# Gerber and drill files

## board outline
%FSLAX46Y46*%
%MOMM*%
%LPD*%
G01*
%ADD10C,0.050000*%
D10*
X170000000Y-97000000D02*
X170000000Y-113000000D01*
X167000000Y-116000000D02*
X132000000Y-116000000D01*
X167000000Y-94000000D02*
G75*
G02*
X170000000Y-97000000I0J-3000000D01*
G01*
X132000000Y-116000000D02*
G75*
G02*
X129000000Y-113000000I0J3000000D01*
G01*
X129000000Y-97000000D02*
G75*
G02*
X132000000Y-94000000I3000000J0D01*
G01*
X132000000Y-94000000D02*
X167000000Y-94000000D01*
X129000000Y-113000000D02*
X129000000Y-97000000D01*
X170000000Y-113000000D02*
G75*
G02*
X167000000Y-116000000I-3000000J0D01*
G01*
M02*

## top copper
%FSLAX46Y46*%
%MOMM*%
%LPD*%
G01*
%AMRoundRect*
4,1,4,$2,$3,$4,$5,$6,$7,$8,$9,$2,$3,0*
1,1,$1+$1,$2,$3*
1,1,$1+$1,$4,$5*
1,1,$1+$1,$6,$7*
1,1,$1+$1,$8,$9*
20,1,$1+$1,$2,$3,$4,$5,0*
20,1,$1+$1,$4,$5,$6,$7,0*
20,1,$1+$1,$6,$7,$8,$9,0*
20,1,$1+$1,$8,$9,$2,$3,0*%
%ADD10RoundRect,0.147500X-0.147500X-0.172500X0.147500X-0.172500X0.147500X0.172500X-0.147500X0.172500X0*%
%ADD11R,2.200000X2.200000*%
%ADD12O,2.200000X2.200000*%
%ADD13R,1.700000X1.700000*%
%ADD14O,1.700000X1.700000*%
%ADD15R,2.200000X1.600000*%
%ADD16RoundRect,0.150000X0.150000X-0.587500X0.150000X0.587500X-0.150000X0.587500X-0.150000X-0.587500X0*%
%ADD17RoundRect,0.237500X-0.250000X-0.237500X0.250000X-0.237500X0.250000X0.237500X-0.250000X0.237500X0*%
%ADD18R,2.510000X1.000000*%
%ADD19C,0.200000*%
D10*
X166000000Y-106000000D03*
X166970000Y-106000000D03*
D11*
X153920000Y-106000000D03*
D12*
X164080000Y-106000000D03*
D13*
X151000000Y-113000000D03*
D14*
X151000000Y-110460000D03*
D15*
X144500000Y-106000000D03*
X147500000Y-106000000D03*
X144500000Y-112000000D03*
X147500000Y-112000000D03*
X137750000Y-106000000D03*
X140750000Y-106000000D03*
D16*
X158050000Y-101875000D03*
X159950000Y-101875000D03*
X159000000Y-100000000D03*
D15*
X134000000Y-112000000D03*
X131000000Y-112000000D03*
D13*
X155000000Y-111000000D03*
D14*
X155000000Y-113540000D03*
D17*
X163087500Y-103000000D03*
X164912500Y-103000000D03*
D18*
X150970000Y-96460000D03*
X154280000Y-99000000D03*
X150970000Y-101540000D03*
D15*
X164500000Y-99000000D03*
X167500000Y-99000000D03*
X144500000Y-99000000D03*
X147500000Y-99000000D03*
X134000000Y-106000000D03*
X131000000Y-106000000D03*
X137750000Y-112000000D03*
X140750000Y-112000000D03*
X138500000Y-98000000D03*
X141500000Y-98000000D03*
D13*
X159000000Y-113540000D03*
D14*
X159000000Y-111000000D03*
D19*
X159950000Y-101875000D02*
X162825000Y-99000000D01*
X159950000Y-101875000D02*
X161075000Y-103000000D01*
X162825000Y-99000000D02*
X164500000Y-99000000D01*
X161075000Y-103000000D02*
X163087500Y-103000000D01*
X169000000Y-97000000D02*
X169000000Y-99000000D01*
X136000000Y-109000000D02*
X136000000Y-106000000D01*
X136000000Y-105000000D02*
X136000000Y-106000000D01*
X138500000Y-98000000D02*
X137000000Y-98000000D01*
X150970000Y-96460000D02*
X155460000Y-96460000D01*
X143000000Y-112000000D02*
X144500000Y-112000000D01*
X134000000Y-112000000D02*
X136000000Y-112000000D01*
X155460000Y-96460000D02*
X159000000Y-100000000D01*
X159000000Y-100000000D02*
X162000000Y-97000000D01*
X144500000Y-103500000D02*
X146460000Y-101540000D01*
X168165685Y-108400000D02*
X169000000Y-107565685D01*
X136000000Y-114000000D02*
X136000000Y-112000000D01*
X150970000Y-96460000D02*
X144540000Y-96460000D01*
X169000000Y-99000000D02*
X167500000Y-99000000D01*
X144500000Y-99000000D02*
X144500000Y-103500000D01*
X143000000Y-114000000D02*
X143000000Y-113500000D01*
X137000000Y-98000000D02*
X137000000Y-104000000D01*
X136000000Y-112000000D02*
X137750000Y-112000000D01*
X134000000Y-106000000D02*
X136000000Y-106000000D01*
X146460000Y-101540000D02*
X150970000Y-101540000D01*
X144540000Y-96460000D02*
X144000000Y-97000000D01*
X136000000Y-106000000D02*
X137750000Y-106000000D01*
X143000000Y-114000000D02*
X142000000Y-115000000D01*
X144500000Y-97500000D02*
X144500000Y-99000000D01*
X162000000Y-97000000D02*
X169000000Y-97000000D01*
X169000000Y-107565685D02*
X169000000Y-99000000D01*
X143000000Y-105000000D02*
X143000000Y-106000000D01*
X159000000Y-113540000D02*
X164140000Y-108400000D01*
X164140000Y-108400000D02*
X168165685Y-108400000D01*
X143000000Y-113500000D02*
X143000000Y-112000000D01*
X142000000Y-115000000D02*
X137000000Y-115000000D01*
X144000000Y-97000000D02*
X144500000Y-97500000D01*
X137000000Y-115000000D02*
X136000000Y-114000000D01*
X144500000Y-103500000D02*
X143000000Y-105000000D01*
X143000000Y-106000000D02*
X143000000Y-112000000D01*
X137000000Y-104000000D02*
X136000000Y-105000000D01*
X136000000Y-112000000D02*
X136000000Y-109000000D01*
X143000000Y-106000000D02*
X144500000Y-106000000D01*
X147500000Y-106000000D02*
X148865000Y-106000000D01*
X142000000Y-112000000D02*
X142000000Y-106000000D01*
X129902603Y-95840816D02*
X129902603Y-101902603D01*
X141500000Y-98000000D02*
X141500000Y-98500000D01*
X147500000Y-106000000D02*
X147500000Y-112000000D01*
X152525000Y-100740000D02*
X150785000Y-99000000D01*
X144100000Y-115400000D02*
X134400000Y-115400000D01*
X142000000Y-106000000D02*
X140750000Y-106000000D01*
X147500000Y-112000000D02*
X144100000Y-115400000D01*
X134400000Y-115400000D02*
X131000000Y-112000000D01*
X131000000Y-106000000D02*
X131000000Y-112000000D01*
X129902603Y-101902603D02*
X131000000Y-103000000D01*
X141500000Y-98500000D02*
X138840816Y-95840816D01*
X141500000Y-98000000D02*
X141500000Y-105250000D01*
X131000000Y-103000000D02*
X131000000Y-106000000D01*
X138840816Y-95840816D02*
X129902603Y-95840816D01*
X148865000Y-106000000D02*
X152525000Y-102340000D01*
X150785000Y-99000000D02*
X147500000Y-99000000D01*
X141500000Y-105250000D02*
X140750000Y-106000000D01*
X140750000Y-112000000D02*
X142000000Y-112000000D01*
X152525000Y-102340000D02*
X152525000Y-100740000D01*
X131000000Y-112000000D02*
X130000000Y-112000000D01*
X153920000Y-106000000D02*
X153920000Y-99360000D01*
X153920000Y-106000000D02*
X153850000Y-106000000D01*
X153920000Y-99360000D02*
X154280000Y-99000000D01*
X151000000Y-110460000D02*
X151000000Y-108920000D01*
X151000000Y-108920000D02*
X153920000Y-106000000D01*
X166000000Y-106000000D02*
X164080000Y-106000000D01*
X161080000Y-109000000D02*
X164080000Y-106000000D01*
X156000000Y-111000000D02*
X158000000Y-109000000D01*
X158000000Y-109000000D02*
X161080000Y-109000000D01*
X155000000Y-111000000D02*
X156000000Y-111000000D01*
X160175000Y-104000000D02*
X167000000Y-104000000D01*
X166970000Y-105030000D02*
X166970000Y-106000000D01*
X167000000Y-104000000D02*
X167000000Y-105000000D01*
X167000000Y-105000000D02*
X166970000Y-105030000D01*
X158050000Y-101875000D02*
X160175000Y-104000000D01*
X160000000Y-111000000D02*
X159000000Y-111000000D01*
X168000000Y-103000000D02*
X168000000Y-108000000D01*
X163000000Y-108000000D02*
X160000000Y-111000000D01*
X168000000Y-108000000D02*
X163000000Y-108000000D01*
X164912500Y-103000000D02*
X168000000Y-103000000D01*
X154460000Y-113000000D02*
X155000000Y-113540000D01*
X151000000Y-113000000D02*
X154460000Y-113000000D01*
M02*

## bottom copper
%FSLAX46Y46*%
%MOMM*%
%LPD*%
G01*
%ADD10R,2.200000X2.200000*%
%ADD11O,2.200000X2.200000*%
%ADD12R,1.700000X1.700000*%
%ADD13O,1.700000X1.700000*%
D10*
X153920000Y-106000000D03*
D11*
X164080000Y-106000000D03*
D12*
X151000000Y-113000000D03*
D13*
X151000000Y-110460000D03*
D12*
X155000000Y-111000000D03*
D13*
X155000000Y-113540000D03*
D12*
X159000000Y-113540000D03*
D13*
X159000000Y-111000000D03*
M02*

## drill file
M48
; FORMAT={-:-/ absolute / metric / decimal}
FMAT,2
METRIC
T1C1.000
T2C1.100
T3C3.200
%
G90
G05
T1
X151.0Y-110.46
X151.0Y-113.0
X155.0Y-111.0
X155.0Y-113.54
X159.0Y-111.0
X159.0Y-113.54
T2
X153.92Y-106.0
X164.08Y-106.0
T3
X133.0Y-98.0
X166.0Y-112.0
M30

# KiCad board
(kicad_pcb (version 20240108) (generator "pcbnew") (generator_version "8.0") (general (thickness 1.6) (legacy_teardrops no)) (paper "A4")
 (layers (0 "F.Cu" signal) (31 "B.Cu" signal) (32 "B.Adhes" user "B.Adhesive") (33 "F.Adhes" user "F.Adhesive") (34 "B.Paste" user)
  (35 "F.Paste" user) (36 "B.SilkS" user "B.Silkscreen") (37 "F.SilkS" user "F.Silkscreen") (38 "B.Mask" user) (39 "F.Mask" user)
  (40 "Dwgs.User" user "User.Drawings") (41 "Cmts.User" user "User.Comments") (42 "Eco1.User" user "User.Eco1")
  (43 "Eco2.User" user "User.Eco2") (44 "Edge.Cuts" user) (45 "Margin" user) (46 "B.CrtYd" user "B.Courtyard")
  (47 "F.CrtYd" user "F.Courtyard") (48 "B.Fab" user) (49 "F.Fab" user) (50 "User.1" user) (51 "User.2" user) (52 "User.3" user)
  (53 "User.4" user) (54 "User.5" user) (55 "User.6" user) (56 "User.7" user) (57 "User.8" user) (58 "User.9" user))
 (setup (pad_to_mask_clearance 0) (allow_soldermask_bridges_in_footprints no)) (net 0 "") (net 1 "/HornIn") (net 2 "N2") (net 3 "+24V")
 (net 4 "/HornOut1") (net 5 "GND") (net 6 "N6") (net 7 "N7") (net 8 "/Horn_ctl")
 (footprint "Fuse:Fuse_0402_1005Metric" (layer "F.Cu") (at 166.485 106)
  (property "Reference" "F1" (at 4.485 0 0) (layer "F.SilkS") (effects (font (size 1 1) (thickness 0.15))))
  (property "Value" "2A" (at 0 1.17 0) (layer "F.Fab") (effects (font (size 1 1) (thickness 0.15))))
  (pad "1" smd roundrect (at -0.485 0) (size 0.59 0.64) (layers "F.Cu" "F.Paste" "F.Mask") (roundrect_rratio 0.25) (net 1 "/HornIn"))
  (pad "2" smd roundrect (at 0.485 0) (size 0.59 0.64) (layers "F.Cu" "F.Paste" "F.Mask") (roundrect_rratio 0.25) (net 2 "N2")))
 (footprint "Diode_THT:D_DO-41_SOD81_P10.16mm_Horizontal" (layer "F.Cu") (at 153.92 106)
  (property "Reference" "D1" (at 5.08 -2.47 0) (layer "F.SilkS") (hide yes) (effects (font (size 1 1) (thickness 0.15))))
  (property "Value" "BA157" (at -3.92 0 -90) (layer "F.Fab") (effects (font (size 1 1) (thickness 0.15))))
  (pad "1" thru_hole rect (at 0 0) (size 2.2 2.2) (drill 1.1) (layers "*.Cu" "*.Mask") (remove_unused_layers no) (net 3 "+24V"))
  (pad "2" thru_hole oval (at 10.16 0) (size 2.2 2.2) (drill 1.1) (layers "*.Cu" "*.Mask") (remove_unused_layers no) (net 1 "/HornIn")))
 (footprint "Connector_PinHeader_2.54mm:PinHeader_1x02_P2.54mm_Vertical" (layer "F.Cu") (at 151 113 180)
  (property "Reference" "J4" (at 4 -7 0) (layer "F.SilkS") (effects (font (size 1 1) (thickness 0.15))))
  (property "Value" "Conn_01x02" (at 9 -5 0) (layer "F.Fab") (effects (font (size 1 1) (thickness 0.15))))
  (pad "1" thru_hole rect (at 0 0 180) (size 1.7 1.7) (drill 1) (layers "*.Cu" "*.Mask") (remove_unused_layers no) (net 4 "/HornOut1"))
  (pad "2" thru_hole oval (at 0 2.54 180) (size 1.7 1.7) (drill 1) (layers "*.Cu" "*.Mask") (remove_unused_layers no) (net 3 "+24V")))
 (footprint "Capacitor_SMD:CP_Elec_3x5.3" (layer "F.Cu") (at 146 106)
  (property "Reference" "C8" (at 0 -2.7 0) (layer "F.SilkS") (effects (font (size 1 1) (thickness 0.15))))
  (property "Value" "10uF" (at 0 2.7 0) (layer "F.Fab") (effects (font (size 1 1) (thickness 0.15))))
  (pad "1" smd rect (at -1.5 0) (size 2.2 1.6) (layers "F.Cu" "F.Paste" "F.Mask") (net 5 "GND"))
  (pad "2" smd rect (at 1.5 0) (size 2.2 1.6) (layers "F.Cu" "F.Paste" "F.Mask") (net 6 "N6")))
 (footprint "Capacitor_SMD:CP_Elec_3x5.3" (layer "F.Cu") (at 146 112)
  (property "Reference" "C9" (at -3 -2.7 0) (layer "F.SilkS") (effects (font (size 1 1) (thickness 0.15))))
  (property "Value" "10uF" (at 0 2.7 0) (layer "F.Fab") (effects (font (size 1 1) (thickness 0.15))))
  (pad "1" smd rect (at -1.5 0) (size 2.2 1.6) (layers "F.Cu" "F.Paste" "F.Mask") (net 5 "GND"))
  (pad "2" smd rect (at 1.5 0) (size 2.2 1.6) (layers "F.Cu" "F.Paste" "F.Mask") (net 6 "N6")))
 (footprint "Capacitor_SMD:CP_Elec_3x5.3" (layer "F.Cu") (at 139.25 106)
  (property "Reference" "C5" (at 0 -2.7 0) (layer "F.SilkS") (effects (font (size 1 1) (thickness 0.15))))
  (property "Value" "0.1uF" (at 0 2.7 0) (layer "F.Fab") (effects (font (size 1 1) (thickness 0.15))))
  (pad "1" smd rect (at -1.5 0) (size 2.2 1.6) (layers "F.Cu" "F.Paste" "F.Mask") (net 5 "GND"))
  (pad "2" smd rect (at 1.5 0) (size 2.2 1.6) (layers "F.Cu" "F.Paste" "F.Mask") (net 6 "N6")))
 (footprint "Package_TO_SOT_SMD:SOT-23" (layer "F.Cu") (at 159 100.9375 90)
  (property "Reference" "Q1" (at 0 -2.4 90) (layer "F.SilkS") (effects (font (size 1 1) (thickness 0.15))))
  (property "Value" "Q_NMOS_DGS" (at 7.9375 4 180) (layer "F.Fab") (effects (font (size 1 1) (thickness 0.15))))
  (pad "1" smd roundrect (at -0.9375 -0.95 90) (size 1.475 0.6) (layers "F.Cu" "F.Paste" "F.Mask") (roundrect_rratio 0.25) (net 2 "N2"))
  (pad "2" smd roundrect (at -0.9375 0.95 90) (size 1.475 0.6) (layers "F.Cu" "F.Paste" "F.Mask") (roundrect_rratio 0.25) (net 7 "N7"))
  (pad "3" smd roundrect (at 0.9375 0 90) (size 1.475 0.6) (layers "F.Cu" "F.Paste" "F.Mask") (roundrect_rratio 0.25) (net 5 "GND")))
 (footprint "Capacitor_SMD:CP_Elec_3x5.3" (layer "F.Cu") (at 132.5 112 180)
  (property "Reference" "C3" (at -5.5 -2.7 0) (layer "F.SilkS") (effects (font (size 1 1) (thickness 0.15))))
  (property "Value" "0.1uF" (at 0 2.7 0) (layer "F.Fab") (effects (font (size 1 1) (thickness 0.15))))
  (pad "1" smd rect (at -1.5 0 180) (size 2.2 1.6) (layers "F.Cu" "F.Paste" "F.Mask") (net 5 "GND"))
  (pad "2" smd rect (at 1.5 0 180) (size 2.2 1.6) (layers "F.Cu" "F.Paste" "F.Mask") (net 6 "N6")))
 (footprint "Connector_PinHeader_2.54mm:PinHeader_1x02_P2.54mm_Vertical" (layer "F.Cu") (at 155 111)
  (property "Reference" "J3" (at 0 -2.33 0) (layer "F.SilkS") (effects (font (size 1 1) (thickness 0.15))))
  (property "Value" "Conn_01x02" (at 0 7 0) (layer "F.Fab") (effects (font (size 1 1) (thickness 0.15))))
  (pad "1" thru_hole rect (at 0 0) (size 1.7 1.7) (drill 1) (layers "*.Cu" "*.Mask") (remove_unused_layers no) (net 1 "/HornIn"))
  (pad "2" thru_hole oval (at 0 2.54) (size 1.7 1.7) (drill 1) (layers "*.Cu" "*.Mask") (remove_unused_layers no) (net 4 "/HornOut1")))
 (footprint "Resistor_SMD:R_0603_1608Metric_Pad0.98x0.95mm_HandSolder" (layer "F.Cu") (at 164 103)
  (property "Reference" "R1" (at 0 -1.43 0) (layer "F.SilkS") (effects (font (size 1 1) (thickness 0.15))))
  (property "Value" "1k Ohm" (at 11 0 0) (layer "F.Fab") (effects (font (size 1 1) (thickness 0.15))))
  (pad "1" smd roundrect (at -0.9125 0) (size 0.975 0.95) (layers "F.Cu" "F.Paste" "F.Mask") (roundrect_rratio 0.25) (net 7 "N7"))
  (pad "2" smd roundrect (at 0.9125 0) (size 0.975 0.95) (layers "F.Cu" "F.Paste" "F.Mask") (roundrect_rratio 0.25) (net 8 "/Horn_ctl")))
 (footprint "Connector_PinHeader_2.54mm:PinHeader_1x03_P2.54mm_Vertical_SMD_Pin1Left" (layer "F.Cu") (at 152.625 99)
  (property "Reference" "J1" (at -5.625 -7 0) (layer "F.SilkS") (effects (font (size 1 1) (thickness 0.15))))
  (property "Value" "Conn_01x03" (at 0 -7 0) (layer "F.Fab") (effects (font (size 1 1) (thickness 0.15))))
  (pad "1" smd rect (at -1.655 -2.54) (size 2.51 1) (layers "F.Cu" "F.Paste" "F.Mask") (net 5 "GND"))
  (pad "2" smd rect (at 1.655 0) (size 2.51 1) (layers "F.Cu" "F.Paste" "F.Mask") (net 3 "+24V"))
  (pad "3" smd rect (at -1.655 2.54) (size 2.51 1) (layers "F.Cu" "F.Paste" "F.Mask") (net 5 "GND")))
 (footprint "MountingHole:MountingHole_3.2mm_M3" (layer "F.Cu") (at 133 98)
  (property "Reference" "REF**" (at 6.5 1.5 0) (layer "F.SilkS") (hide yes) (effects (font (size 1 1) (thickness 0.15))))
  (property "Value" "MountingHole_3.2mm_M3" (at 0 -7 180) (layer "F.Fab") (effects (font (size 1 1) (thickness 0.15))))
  (pad "" np_thru_hole circle (at 0 0) (size 3.2 3.2) (drill 3.2) (layers "*.Cu" "*.Mask")))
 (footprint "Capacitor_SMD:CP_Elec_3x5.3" (layer "F.Cu") (at 166 99)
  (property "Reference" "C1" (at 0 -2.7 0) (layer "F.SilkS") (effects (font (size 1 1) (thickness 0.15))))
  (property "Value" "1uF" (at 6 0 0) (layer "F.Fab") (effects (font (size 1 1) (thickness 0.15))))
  (pad "1" smd rect (at -1.5 0) (size 2.2 1.6) (layers "F.Cu" "F.Paste" "F.Mask") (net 7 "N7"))
  (pad "2" smd rect (at 1.5 0) (size 2.2 1.6) (layers "F.Cu" "F.Paste" "F.Mask") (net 5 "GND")))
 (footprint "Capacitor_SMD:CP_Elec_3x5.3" (layer "F.Cu") (at 146 99)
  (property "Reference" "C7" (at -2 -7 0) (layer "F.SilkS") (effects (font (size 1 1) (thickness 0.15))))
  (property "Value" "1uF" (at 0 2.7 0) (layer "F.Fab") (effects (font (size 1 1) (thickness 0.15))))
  (pad "1" smd rect (at -1.5 0) (size 2.2 1.6) (layers "F.Cu" "F.Paste" "F.Mask") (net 5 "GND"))
  (pad "2" smd rect (at 1.5 0) (size 2.2 1.6) (layers "F.Cu" "F.Paste" "F.Mask") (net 6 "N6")))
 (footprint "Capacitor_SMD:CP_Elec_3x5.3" (layer "F.Cu") (at 132.5 106 180)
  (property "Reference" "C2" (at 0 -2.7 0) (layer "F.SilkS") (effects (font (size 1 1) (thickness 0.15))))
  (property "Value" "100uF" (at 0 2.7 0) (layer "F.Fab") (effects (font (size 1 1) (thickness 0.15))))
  (pad "1" smd rect (at -1.5 0 180) (size 2.2 1.6) (layers "F.Cu" "F.Paste" "F.Mask") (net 5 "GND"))
  (pad "2" smd rect (at 1.5 0 180) (size 2.2 1.6) (layers "F.Cu" "F.Paste" "F.Mask") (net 6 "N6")))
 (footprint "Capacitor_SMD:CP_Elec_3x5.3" (layer "F.Cu") (at 139.25 112)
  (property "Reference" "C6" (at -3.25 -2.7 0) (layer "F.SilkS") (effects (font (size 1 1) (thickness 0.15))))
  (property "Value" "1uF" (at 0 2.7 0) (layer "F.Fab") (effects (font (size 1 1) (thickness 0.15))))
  (pad "1" smd rect (at -1.5 0) (size 2.2 1.6) (layers "F.Cu" "F.Paste" "F.Mask") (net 5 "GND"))
  (pad "2" smd rect (at 1.5 0) (size 2.2 1.6) (layers "F.Cu" "F.Paste" "F.Mask") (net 6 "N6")))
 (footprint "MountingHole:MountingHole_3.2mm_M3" (layer "F.Cu") (at 166 112)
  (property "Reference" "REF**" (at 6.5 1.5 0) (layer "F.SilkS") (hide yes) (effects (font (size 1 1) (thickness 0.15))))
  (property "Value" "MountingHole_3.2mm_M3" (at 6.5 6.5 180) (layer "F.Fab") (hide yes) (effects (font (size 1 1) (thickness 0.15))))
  (pad "" np_thru_hole circle (at 0 0) (size 3.2 3.2) (drill 3.2) (layers "*.Cu" "*.Mask")))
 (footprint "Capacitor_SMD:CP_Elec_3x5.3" (layer "F.Cu") (at 140 98)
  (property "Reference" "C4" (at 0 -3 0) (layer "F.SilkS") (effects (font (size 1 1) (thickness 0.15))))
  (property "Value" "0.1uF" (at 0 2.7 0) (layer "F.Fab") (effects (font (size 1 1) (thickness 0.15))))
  (pad "1" smd rect (at -1.5 0) (size 2.2 1.6) (layers "F.Cu" "F.Paste" "F.Mask") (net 5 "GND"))
  (pad "2" smd rect (at 1.5 0) (size 2.2 1.6) (layers "F.Cu" "F.Paste" "F.Mask") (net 6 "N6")))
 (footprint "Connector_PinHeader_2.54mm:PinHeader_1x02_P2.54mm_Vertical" (layer "F.Cu") (at 159 113.54 180)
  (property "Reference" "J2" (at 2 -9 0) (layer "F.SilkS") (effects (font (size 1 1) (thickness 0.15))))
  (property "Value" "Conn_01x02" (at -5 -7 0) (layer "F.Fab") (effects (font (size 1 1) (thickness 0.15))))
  (pad "1" thru_hole rect (at 0 0 180) (size 1.7 1.7) (drill 1) (layers "*.Cu" "*.Mask") (remove_unused_layers no) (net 5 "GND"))
  (pad "2" thru_hole oval (at 0 2.54 180) (size 1.7 1.7) (drill 1) (layers "*.Cu" "*.Mask") (remove_unused_layers no) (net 8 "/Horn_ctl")))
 (gr_line (start 170 97) (end 170 113) (stroke (width 0.05) (type default)) (layer "Edge.Cuts"))
 (gr_line (start 167 116) (end 132 116) (stroke (width 0.05) (type default)) (layer "Edge.Cuts"))
 (gr_arc (start 167 94) (mid 169.12132 94.87868) (end 170 97) (stroke (width 0.05) (type default)) (layer "Edge.Cuts"))
 (gr_arc (start 132 116) (mid 129.87868 115.12132) (end 129 113) (stroke (width 0.05) (type default)) (layer "Edge.Cuts"))
 (gr_arc (start 129 97) (mid 129.87868 94.87868) (end 132 94) (stroke (width 0.05) (type default)) (layer "Edge.Cuts"))
 (gr_line (start 132 94) (end 167 94) (stroke (width 0.05) (type default)) (layer "Edge.Cuts"))
 (gr_line (start 129 113) (end 129 97) (stroke (width 0.05) (type default)) (layer "Edge.Cuts"))
 (gr_arc (start 170 113) (mid 169.12132 115.12132) (end 167 116) (stroke (width 0.05) (type default)) (layer "Edge.Cuts"))
 (segment (start 159.95 101.875) (end 162.825 99) (width 0.2) (layer "F.Cu") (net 7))
 (segment (start 159.95 101.875) (end 161.075 103) (width 0.2) (layer "F.Cu") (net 7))
 (segment (start 162.825 99) (end 164.5 99) (width 0.2) (layer "F.Cu") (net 7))
 (segment (start 161.075 103) (end 163.0875 103) (width 0.2) (layer "F.Cu") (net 7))
 (segment (start 169 97) (end 169 99) (width 0.2) (layer "F.Cu") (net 5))
 (segment (start 136 109) (end 136 106) (width 0.2) (layer "F.Cu") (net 5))
 (segment (start 136 105) (end 136 106) (width 0.2) (layer "F.Cu") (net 5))
 (segment (start 138.5 98) (end 137 98) (width 0.2) (layer "F.Cu") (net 5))
 (segment (start 150.97 96.46) (end 155.46 96.46) (width 0.2) (layer "F.Cu") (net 5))
 (segment (start 143 112) (end 144.5 112) (width 0.2) (layer "F.Cu") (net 5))
 (segment (start 134 112) (end 136 112) (width 0.2) (layer "F.Cu") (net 5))
 (segment (start 155.46 96.46) (end 159 100) (width 0.2) (layer "F.Cu") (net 5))
 (segment (start 159 100) (end 162 97) (width 0.2) (layer "F.Cu") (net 5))
 (segment (start 144.5 103.5) (end 146.46 101.54) (width 0.2) (layer "F.Cu") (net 5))
 (segment (start 168.165685 108.4) (end 169 107.565685) (width 0.2) (layer "F.Cu") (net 5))
 (segment (start 136 114) (end 136 112) (width 0.2) (layer "F.Cu") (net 5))
 (segment (start 150.97 96.46) (end 144.54 96.46) (width 0.2) (layer "F.Cu") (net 5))
 (segment (start 169 99) (end 167.5 99) (width 0.2) (layer "F.Cu") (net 5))
 (segment (start 144.5 99) (end 144.5 103.5) (width 0.2) (layer "F.Cu") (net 5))
 (segment (start 143 114) (end 143 113.5) (width 0.2) (layer "F.Cu") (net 5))
 (segment (start 137 98) (end 137 104) (width 0.2) (layer "F.Cu") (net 5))
 (segment (start 136 112) (end 137.75 112) (width 0.2) (layer "F.Cu") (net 5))
 (segment (start 134 106) (end 136 106) (width 0.2) (layer "F.Cu") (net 5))
 (segment (start 146.46 101.54) (end 150.97 101.54) (width 0.2) (layer "F.Cu") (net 5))
 (segment (start 144.54 96.46) (end 144 97) (width 0.2) (layer "F.Cu") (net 5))
 (segment (start 136 106) (end 137.75 106) (width 0.2) (layer "F.Cu") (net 5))
 (segment (start 143 114) (end 142 115) (width 0.2) (layer "F.Cu") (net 5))
 (segment (start 144.5 97.5) (end 144.5 99) (width 0.2) (layer "F.Cu") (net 5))
 (segment (start 162 97) (end 169 97) (width 0.2) (layer "F.Cu") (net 5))
 (segment (start 169 107.565685) (end 169 99) (width 0.2) (layer "F.Cu") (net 5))
 (segment (start 143 105) (end 143 106) (width 0.2) (layer "F.Cu") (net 5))
 (segment (start 159 113.54) (end 164.14 108.4) (width 0.2) (layer "F.Cu") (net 5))
 (segment (start 164.14 108.4) (end 168.165685 108.4) (width 0.2) (layer "F.Cu") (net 5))
 (segment (start 143 113.5) (end 143 112) (width 0.2) (layer "F.Cu") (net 5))
 (segment (start 142 115) (end 137 115) (width 0.2) (layer "F.Cu") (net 5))
 (segment (start 144 97) (end 144.5 97.5) (width 0.2) (layer "F.Cu") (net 5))
 (segment (start 137 115) (end 136 114) (width 0.2) (layer "F.Cu") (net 5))
 (segment (start 144.5 103.5) (end 143 105) (width 0.2) (layer "F.Cu") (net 5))
 (segment (start 143 106) (end 143 112) (width 0.2) (layer "F.Cu") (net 5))
 (segment (start 137 104) (end 136 105) (width 0.2) (layer "F.Cu") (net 5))
 (segment (start 136 112) (end 136 109) (width 0.2) (layer "F.Cu") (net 5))
 (segment (start 143 106) (end 144.5 106) (width 0.2) (layer "F.Cu") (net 5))
 (segment (start 147.5 106) (end 148.865 106) (width 0.2) (layer "F.Cu") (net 6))
 (segment (start 142 112) (end 142 106) (width 0.2) (layer "F.Cu") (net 6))
 (segment (start 129.902603 95.840816) (end 129.902603 101.902603) (width 0.2) (layer "F.Cu") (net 6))
 (segment (start 141.5 98) (end 141.5 98.5) (width 0.2) (layer "F.Cu") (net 6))
 (segment (start 147.5 106) (end 147.5 112) (width 0.2) (layer "F.Cu") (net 6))
 (segment (start 152.525 100.74) (end 150.785 99) (width 0.2) (layer "F.Cu") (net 6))
 (segment (start 144.1 115.4) (end 134.4 115.4) (width 0.2) (layer "F.Cu") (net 6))
 (segment (start 142 106) (end 140.75 106) (width 0.2) (layer "F.Cu") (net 6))
 (segment (start 147.5 112) (end 144.1 115.4) (width 0.2) (layer "F.Cu") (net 6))
 (segment (start 134.4 115.4) (end 131 112) (width 0.2) (layer "F.Cu") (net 6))
 (segment (start 131 106) (end 131 112) (width 0.2) (layer "F.Cu") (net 6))
 (segment (start 129.902603 101.902603) (end 131 103) (width 0.2) (layer "F.Cu") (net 6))
 (segment (start 141.5 98.5) (end 138.840816 95.840816) (width 0.2) (layer "F.Cu") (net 6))
 (segment (start 141.5 98) (end 141.5 105.25) (width 0.2) (layer "F.Cu") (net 6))
 (segment (start 131 103) (end 131 106) (width 0.2) (layer "F.Cu") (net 6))
 (segment (start 138.840816 95.840816) (end 129.902603 95.840816) (width 0.2) (layer "F.Cu") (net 6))
 (segment (start 148.865 106) (end 152.525 102.34) (width 0.2) (layer "F.Cu") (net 6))
 (segment (start 150.785 99) (end 147.5 99) (width 0.2) (layer "F.Cu") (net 6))
 (segment (start 141.5 105.25) (end 140.75 106) (width 0.2) (layer "F.Cu") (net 6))
 (segment (start 140.75 112) (end 142 112) (width 0.2) (layer "F.Cu") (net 6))
 (segment (start 152.525 102.34) (end 152.525 100.74) (width 0.2) (layer "F.Cu") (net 6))
 (segment (start 131 112) (end 130 112) (width 0.2) (layer "F.Cu") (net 6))
 (segment (start 153.92 106) (end 153.92 99.36) (width 0.2) (layer "F.Cu") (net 3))
 (segment (start 153.92 106) (end 153.85 106) (width 0.2) (layer "F.Cu") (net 3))
 (segment (start 153.92 99.36) (end 154.28 99) (width 0.2) (layer "F.Cu") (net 3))
 (segment (start 151 110.46) (end 151 108.92) (width 0.2) (layer "F.Cu") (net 3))
 (segment (start 151 108.92) (end 153.92 106) (width 0.2) (layer "F.Cu") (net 3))
 (segment (start 166 106) (end 164.08 106) (width 0.2) (layer "F.Cu") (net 1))
 (segment (start 161.08 109) (end 164.08 106) (width 0.2) (layer "F.Cu") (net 1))
 (segment (start 156 111) (end 158 109) (width 0.2) (layer "F.Cu") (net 1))
 (segment (start 158 109) (end 161.08 109) (width 0.2) (layer "F.Cu") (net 1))
 (segment (start 155 111) (end 156 111) (width 0.2) (layer "F.Cu") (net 1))
 (segment (start 160.175 104) (end 167 104) (width 0.2) (layer "F.Cu") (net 2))
 (segment (start 166.97 105.03) (end 166.97 106) (width 0.2) (layer "F.Cu") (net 2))
 (segment (start 167 104) (end 167 105) (width 0.2) (layer "F.Cu") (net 2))
 (segment (start 167 105) (end 166.97 105.03) (width 0.2) (layer "F.Cu") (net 2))
 (segment (start 158.05 101.875) (end 160.175 104) (width 0.2) (layer "F.Cu") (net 2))
 (segment (start 160 111) (end 159 111) (width 0.2) (layer "F.Cu") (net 8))
 (segment (start 168 103) (end 168 108) (width 0.2) (layer "F.Cu") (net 8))
 (segment (start 163 108) (end 160 111) (width 0.2) (layer "F.Cu") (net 8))
 (segment (start 168 108) (end 163 108) (width 0.2) (layer "F.Cu") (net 8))
 (segment (start 164.9125 103) (end 168 103) (width 0.2) (layer "F.Cu") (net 8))
 (segment (start 154.46 113) (end 155 113.54) (width 0.2) (layer "F.Cu") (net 4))
 (segment (start 151 113) (end 154.46 113) (width 0.2) (layer "F.Cu") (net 4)))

